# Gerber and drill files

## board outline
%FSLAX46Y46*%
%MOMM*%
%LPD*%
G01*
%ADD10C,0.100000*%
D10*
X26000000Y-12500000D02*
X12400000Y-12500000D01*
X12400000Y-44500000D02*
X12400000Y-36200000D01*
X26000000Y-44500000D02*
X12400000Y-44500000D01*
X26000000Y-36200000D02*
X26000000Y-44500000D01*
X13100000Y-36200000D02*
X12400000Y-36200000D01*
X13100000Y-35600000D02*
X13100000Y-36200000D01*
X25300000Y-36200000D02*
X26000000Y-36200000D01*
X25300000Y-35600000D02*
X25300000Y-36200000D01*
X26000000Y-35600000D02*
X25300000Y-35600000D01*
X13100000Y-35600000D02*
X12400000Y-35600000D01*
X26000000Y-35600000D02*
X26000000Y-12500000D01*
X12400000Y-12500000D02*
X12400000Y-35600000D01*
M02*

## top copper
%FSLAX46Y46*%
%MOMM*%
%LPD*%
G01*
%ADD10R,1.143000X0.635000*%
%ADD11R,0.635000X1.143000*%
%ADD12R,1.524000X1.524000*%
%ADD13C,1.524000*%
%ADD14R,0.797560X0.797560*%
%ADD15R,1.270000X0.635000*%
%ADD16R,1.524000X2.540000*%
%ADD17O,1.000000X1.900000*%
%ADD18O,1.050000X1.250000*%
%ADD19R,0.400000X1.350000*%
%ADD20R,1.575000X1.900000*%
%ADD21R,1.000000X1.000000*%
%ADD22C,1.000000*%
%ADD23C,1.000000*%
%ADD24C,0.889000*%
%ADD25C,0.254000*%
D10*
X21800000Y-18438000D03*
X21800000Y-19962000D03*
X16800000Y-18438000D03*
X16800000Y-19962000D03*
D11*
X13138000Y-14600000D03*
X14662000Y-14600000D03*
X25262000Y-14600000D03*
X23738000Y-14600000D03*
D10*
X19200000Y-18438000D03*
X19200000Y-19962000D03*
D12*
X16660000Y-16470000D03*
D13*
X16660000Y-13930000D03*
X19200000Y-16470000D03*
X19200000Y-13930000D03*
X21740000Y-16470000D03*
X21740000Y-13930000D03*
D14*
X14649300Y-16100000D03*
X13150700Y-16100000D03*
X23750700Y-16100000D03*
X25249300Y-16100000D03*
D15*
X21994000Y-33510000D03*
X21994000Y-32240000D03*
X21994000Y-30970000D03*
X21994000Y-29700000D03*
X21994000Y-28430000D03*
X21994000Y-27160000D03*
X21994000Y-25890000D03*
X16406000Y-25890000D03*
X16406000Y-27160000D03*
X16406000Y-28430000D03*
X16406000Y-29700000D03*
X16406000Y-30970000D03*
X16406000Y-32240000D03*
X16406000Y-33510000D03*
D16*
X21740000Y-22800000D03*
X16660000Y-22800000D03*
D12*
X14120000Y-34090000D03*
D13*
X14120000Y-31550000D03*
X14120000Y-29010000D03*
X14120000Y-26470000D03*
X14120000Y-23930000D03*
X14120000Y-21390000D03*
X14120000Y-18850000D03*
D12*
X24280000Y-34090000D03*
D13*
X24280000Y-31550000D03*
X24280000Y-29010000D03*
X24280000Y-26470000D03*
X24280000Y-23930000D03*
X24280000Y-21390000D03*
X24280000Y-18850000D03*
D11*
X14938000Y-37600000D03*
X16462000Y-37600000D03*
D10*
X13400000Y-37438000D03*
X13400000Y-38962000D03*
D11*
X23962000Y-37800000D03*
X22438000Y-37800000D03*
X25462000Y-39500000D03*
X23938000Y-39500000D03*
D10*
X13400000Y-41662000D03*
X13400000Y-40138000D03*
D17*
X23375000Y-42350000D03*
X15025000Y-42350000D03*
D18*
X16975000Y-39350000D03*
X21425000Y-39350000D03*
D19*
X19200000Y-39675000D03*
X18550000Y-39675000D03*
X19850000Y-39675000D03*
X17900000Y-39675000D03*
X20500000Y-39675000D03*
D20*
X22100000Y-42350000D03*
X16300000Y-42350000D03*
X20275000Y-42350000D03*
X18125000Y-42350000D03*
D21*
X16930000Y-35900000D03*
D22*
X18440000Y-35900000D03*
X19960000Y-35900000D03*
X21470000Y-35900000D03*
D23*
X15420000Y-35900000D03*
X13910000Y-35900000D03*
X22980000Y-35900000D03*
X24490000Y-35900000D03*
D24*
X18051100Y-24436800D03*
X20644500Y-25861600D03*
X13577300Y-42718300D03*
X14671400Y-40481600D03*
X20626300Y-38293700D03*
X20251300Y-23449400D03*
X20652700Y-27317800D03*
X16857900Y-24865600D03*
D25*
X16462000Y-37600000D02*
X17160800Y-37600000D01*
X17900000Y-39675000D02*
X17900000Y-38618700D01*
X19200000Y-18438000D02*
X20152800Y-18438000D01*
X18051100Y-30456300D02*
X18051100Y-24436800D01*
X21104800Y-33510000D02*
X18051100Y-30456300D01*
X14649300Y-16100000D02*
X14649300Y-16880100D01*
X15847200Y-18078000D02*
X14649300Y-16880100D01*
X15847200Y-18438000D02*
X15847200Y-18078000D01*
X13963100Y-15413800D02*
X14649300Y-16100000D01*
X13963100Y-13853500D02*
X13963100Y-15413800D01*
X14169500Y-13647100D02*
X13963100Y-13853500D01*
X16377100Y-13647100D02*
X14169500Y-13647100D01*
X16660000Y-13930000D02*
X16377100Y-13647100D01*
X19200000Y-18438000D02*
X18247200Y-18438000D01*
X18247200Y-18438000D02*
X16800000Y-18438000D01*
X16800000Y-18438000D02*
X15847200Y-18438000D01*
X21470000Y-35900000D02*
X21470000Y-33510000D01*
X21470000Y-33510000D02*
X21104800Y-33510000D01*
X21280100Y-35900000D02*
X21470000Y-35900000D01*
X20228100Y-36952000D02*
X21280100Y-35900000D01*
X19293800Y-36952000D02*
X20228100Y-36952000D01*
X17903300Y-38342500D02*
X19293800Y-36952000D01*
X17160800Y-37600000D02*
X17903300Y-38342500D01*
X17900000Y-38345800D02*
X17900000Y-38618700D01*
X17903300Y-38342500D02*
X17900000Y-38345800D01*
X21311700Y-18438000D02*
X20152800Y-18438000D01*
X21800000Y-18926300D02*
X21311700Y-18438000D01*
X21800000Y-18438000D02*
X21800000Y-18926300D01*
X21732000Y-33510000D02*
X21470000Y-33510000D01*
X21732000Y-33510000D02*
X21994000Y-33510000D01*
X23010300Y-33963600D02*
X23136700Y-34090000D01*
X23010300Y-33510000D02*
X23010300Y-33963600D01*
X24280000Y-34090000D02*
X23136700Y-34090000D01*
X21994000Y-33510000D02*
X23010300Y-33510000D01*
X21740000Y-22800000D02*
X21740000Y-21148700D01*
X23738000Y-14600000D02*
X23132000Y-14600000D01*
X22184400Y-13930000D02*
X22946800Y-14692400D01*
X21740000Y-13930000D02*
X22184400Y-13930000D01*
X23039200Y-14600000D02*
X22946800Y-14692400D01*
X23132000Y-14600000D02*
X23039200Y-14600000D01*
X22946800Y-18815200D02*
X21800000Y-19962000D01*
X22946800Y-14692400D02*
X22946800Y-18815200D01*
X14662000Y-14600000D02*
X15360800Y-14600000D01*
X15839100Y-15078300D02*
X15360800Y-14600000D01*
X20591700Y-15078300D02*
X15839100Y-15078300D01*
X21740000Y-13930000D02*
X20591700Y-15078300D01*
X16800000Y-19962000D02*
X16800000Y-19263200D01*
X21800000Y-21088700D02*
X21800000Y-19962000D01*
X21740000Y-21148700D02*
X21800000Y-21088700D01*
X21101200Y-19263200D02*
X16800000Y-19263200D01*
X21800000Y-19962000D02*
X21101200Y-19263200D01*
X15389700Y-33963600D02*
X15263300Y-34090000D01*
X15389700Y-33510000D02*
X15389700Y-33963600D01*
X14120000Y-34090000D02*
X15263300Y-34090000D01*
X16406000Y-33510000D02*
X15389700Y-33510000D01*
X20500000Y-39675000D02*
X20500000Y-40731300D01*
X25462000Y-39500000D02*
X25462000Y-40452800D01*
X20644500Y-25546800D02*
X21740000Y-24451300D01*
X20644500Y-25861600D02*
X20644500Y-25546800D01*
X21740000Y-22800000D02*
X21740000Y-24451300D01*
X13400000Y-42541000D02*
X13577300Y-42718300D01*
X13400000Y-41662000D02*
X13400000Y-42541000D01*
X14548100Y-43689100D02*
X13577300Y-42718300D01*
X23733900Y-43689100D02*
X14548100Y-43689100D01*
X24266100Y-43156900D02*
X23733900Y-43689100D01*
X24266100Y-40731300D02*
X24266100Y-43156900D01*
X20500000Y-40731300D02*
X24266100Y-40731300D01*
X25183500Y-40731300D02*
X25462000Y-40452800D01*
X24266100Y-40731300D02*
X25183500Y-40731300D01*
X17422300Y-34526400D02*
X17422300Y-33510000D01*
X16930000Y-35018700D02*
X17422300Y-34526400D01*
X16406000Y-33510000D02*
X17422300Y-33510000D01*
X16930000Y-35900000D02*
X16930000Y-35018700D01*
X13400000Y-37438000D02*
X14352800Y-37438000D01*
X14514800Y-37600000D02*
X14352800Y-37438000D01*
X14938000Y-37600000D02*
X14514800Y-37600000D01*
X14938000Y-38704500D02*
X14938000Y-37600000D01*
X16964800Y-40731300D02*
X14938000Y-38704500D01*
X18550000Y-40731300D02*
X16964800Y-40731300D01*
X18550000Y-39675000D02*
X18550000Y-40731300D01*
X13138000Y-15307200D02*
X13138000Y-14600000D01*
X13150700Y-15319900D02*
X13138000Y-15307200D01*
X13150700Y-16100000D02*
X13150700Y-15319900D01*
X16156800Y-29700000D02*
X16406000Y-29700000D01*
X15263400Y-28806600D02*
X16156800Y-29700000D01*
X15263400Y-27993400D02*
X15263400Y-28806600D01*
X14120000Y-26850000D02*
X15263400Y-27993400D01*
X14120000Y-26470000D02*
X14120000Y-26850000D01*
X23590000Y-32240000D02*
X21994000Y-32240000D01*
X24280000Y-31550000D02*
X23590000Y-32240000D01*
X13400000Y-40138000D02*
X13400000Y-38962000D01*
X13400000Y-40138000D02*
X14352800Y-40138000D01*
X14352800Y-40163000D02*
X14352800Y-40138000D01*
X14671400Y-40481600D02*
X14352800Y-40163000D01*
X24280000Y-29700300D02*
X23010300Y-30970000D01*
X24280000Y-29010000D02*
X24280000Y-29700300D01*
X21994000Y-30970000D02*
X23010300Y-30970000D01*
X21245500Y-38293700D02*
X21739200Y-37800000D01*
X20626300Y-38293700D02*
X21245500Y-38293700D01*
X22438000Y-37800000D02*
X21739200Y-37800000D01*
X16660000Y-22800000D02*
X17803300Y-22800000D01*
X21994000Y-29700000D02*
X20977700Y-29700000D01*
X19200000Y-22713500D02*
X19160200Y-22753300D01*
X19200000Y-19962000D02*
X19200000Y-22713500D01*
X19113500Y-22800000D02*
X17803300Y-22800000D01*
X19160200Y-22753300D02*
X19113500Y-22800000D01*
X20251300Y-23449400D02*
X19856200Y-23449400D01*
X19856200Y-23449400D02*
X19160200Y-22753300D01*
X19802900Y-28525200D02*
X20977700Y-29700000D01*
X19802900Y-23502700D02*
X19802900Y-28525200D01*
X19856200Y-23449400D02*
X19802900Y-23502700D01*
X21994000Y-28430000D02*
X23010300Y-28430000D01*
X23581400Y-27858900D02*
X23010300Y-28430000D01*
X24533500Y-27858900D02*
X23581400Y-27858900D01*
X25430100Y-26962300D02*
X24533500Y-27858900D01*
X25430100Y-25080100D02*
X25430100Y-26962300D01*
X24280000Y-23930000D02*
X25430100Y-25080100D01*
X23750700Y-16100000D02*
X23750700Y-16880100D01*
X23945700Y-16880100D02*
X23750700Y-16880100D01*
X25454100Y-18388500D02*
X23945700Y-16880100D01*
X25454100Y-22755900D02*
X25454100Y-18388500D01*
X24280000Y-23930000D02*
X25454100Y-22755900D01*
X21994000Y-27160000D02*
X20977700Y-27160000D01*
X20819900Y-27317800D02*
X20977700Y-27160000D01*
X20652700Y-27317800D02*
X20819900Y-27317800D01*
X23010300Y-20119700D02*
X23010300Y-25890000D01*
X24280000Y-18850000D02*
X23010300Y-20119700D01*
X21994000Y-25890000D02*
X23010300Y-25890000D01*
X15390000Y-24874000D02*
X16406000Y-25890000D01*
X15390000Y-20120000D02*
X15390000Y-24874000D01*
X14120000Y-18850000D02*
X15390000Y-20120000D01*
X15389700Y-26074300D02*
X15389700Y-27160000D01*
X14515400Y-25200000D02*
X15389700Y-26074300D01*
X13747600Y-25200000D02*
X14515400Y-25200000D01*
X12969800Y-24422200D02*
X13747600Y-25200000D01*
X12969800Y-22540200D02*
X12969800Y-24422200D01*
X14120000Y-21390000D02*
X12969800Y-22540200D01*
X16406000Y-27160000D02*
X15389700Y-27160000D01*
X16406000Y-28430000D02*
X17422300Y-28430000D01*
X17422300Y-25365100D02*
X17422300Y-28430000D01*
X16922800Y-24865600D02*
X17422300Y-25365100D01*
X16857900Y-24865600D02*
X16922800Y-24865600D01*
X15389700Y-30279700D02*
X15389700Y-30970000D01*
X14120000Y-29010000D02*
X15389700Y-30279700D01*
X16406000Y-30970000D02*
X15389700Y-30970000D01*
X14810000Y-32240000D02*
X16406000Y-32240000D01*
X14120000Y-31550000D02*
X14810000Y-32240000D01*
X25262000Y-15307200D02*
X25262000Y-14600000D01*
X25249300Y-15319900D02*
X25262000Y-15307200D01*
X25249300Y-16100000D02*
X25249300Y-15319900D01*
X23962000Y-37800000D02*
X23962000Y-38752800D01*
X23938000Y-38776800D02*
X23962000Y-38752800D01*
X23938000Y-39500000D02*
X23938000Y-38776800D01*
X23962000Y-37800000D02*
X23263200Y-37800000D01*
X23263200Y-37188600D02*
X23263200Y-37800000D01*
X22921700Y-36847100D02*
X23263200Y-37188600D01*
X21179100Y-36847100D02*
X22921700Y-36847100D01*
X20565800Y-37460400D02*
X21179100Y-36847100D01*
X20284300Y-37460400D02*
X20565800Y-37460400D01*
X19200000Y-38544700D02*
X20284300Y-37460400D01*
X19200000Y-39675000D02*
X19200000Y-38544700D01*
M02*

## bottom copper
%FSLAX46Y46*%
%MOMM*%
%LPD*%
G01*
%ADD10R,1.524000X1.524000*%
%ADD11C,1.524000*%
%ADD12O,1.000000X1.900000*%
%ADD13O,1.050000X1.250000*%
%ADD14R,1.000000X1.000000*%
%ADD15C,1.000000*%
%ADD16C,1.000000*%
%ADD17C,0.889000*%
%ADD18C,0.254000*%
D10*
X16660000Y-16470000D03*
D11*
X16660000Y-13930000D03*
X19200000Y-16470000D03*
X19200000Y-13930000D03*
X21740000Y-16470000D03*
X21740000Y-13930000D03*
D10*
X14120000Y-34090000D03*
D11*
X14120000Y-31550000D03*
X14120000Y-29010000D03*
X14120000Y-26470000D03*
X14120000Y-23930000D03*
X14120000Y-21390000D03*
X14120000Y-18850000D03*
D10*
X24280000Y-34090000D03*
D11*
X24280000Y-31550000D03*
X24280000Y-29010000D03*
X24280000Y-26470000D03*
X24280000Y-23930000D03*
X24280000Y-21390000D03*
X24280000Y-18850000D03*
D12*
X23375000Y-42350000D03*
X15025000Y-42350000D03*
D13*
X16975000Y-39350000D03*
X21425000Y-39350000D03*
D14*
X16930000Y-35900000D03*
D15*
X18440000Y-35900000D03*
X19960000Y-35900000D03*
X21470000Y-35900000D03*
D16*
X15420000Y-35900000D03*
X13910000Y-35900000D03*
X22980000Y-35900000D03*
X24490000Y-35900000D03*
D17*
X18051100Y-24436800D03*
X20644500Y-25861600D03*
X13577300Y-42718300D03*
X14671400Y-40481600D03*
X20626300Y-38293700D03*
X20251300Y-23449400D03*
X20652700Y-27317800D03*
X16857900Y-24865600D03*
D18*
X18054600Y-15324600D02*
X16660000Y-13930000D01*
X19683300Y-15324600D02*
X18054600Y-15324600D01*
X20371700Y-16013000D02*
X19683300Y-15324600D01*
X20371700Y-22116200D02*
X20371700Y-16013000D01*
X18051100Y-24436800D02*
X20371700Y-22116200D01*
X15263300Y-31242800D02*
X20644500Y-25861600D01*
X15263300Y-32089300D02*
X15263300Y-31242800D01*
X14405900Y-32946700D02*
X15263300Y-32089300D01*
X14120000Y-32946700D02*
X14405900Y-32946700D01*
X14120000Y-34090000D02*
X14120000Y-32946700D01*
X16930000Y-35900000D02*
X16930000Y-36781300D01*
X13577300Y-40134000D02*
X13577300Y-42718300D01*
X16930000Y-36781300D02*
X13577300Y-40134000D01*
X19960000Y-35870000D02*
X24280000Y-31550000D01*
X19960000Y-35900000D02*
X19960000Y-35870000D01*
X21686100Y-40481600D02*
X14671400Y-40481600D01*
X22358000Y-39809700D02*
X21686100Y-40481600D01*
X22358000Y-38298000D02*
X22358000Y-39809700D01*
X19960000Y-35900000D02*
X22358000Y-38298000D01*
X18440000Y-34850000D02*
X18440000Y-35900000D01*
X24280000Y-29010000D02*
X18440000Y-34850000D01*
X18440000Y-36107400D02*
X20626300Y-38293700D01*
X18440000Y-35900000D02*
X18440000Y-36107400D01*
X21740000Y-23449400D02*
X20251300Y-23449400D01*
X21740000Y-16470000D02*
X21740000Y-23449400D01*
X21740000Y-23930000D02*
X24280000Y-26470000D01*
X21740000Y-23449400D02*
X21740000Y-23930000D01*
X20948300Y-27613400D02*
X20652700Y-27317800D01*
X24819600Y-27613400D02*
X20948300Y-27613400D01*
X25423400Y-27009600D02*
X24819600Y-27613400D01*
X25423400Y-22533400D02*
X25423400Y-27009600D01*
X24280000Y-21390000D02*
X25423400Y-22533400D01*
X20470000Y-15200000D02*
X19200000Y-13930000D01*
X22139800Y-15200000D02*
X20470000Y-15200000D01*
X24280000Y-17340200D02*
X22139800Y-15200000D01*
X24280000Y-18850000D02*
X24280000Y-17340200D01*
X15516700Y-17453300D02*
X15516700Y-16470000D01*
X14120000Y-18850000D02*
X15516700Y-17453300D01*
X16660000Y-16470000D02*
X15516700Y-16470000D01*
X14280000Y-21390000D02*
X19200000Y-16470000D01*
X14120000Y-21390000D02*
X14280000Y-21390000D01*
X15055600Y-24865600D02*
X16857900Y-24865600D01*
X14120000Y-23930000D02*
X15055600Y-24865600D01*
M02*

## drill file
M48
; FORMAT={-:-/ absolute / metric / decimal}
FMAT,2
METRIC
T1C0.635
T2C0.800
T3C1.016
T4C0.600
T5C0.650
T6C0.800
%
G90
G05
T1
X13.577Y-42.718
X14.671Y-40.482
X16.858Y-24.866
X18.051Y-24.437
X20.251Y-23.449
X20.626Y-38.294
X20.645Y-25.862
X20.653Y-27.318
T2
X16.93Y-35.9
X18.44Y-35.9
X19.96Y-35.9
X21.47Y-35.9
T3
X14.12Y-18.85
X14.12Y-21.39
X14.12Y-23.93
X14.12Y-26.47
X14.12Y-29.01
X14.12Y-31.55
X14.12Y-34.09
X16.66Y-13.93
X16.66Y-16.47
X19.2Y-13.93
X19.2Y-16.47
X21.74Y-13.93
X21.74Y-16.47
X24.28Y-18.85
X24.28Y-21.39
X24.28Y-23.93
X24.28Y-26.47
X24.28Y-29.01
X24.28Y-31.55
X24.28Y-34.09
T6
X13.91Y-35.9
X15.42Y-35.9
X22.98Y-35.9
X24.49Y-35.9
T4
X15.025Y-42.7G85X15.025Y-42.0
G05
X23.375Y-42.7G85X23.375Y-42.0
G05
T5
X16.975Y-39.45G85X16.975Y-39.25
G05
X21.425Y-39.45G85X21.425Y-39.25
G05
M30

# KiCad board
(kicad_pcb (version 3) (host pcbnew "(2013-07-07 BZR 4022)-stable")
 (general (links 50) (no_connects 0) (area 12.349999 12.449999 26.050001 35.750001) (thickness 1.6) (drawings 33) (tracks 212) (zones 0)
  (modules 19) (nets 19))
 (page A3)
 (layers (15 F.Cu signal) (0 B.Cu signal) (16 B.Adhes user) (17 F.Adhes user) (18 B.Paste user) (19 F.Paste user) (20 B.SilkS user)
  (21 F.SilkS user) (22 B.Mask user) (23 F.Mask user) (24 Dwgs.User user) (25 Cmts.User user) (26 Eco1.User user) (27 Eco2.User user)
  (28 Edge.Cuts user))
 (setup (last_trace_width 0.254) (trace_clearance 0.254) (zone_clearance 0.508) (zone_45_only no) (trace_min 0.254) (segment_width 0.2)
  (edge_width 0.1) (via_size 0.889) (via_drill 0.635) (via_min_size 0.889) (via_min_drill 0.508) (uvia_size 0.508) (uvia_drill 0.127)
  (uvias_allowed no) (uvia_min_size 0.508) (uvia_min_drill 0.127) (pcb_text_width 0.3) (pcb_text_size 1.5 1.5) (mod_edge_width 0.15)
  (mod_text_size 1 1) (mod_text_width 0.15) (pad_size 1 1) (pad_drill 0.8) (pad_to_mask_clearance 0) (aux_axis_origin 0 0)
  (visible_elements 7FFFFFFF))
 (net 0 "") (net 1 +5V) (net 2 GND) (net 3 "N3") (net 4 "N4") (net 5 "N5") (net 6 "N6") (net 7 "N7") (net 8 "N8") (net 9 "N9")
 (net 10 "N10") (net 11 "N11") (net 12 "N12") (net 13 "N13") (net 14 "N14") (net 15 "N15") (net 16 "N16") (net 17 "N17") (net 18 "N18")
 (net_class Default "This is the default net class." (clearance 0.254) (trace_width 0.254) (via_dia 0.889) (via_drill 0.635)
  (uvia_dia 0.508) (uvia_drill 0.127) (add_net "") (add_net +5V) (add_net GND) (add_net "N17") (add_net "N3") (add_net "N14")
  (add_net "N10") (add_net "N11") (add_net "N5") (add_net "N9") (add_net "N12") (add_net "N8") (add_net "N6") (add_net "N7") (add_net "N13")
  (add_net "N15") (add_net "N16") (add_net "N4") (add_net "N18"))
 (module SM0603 (layer F.Cu) (at 21.8 19.2 270)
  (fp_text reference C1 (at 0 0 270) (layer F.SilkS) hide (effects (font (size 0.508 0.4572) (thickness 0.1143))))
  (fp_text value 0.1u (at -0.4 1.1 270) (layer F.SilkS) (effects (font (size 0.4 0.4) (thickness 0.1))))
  (pad 1 smd rect (at -0.762 0 270) (size 0.635 1.143) (layers F.Cu F.Paste F.Mask) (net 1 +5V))
  (pad 2 smd rect (at 0.762 0 270) (size 0.635 1.143) (layers F.Cu F.Paste F.Mask) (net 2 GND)))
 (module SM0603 (layer F.Cu) (at 16.8 19.2 270)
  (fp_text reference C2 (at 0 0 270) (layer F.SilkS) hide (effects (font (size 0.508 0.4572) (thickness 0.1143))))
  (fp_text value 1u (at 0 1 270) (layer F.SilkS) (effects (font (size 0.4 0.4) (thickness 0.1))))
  (pad 1 smd rect (at -0.762 0 270) (size 0.635 1.143) (layers F.Cu F.Paste F.Mask) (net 1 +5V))
  (pad 2 smd rect (at 0.762 0 270) (size 0.635 1.143) (layers F.Cu F.Paste F.Mask) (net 2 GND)))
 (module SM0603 (layer F.Cu) (at 13.9 14.6)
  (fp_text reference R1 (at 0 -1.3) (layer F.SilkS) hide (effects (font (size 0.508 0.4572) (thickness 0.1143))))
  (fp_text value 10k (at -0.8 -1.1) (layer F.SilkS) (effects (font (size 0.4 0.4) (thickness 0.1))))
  (pad 1 smd rect (at -0.762 0) (size 0.635 1.143) (layers F.Cu F.Paste F.Mask) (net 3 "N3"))
  (pad 2 smd rect (at 0.762 0) (size 0.635 1.143) (layers F.Cu F.Paste F.Mask) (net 2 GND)))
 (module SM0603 (layer F.Cu) (at 24.5 14.6 180)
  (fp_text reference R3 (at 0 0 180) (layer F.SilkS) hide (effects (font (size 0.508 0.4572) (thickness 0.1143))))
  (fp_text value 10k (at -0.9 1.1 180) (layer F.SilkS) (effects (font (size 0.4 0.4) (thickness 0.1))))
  (pad 1 smd rect (at -0.762 0 180) (size 0.635 1.143) (layers F.Cu F.Paste F.Mask) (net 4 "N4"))
  (pad 2 smd rect (at 0.762 0 180) (size 0.635 1.143) (layers F.Cu F.Paste F.Mask) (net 2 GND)))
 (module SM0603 (layer F.Cu) (at 19.2 19.2 270)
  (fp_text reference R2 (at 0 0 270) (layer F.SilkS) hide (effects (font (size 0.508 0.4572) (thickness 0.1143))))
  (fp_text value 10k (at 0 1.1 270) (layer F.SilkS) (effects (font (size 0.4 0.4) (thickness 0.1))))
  (pad 1 smd rect (at -0.762 0 270) (size 0.635 1.143) (layers F.Cu F.Paste F.Mask) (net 1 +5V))
  (pad 2 smd rect (at 0.762 0 270) (size 0.635 1.143) (layers F.Cu F.Paste F.Mask) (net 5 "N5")))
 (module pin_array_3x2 (layer F.Cu) (at 19.2 15.2)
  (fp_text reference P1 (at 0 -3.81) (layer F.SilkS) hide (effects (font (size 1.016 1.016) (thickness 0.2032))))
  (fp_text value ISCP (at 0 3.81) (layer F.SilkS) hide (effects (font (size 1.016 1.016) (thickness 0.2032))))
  (pad 1 thru_hole rect (at -2.54 1.27) (size 1.524 1.524) (drill 1.016) (layers *.Cu *.Mask F.SilkS) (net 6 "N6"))
  (pad 2 thru_hole circle (at -2.54 -1.27) (size 1.524 1.524) (drill 1.016) (layers *.Cu *.Mask F.SilkS) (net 1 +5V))
  (pad 3 thru_hole circle (at 0 1.27) (size 1.524 1.524) (drill 1.016) (layers *.Cu *.Mask F.SilkS) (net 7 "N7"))
  (pad 4 thru_hole circle (at 0 -1.27) (size 1.524 1.524) (drill 1.016) (layers *.Cu *.Mask F.SilkS) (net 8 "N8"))
  (pad 5 thru_hole circle (at 2.54 1.27) (size 1.524 1.524) (drill 1.016) (layers *.Cu *.Mask F.SilkS) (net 5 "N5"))
  (pad 6 thru_hole circle (at 2.54 -1.27) (size 1.524 1.524) (drill 1.016) (layers *.Cu *.Mask F.SilkS) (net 2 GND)))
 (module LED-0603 (layer F.Cu) (at 13.9 16.1 180)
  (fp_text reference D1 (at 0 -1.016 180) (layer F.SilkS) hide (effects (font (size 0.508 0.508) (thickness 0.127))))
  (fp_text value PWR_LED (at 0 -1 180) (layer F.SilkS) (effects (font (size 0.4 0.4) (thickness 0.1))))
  (pad 1 smd rect (at -0.7493 0 180) (size 0.79756 0.79756) (layers F.Cu F.Paste F.Mask) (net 1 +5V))
  (pad 2 smd rect (at 0.7493 0 180) (size 0.79756 0.79756) (layers F.Cu F.Paste F.Mask) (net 3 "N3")))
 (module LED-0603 (layer F.Cu) (at 24.5 16.1)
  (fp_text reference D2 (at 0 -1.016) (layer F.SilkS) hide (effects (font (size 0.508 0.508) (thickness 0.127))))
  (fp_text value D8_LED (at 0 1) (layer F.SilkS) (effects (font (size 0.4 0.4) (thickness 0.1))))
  (pad 1 smd rect (at -0.7493 0) (size 0.79756 0.79756) (layers F.Cu F.Paste F.Mask) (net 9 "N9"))
  (pad 2 smd rect (at 0.7493 0) (size 0.79756 0.79756) (layers F.Cu F.Paste F.Mask) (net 4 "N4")))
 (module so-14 (layer F.Cu) (at 19.2 29.7 90)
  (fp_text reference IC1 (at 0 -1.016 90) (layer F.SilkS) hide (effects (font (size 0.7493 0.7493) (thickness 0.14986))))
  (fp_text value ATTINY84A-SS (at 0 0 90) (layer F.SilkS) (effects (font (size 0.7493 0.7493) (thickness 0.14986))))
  (pad 1 smd rect (at -3.81 2.794 90) (size 0.635 1.27) (layers F.Cu F.Paste F.Mask) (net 1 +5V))
  (pad 2 smd rect (at -2.54 2.794 90) (size 0.635 1.27) (layers F.Cu F.Paste F.Mask) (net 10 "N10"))
  (pad 3 smd rect (at -1.27 2.794 90) (size 0.635 1.27) (layers F.Cu F.Paste F.Mask) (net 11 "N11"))
  (pad 4 smd rect (at 0 2.794 90) (size 0.635 1.27) (layers F.Cu F.Paste F.Mask) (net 5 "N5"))
  (pad 5 smd rect (at 1.27 2.794 90) (size 0.635 1.27) (layers F.Cu F.Paste F.Mask) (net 9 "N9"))
  (pad 6 smd rect (at 2.54 2.794 90) (size 0.635 1.27) (layers F.Cu F.Paste F.Mask) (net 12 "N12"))
  (pad 7 smd rect (at 3.81 2.794 90) (size 0.635 1.27) (layers F.Cu F.Paste F.Mask) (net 8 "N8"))
  (pad 8 smd rect (at 3.81 -2.794 90) (size 0.635 1.27) (layers F.Cu F.Paste F.Mask) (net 6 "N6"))
  (pad 9 smd rect (at 2.54 -2.794 90) (size 0.635 1.27) (layers F.Cu F.Paste F.Mask) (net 7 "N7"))
  (pad 10 smd rect (at 1.27 -2.794 90) (size 0.635 1.27) (layers F.Cu F.Paste F.Mask) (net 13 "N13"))
  (pad 11 smd rect (at 0 -2.794 90) (size 0.635 1.27) (layers F.Cu F.Paste F.Mask) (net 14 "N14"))
  (pad 12 smd rect (at -1.27 -2.794 90) (size 0.635 1.27) (layers F.Cu F.Paste F.Mask) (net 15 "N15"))
  (pad 13 smd rect (at -2.54 -2.794 90) (size 0.635 1.27) (layers F.Cu F.Paste F.Mask) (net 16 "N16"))
  (pad 14 smd rect (at -3.81 -2.794 90) (size 0.635 1.27) (layers F.Cu F.Paste F.Mask) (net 2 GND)))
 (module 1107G (layer F.Cu) (at 19.2 22.8)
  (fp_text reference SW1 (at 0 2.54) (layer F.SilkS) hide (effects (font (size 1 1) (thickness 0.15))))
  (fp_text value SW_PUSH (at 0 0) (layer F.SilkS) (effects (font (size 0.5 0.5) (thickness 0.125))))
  (pad 1 smd rect (at 2.54 0) (size 1.524 2.54) (layers F.Cu F.Paste F.Mask) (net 2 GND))
  (pad 2 smd rect (at -2.54 0) (size 1.524 2.54) (layers F.Cu F.Paste F.Mask) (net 5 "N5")))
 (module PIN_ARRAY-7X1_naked (layer F.Cu) (at 14.12 26.47 90)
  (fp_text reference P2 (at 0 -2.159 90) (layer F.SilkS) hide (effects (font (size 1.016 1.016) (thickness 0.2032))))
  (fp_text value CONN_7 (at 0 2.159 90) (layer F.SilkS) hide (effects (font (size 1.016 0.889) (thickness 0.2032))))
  (pad 1 thru_hole rect (at -7.62 0 90) (size 1.524 1.524) (drill 1.016) (layers *.Cu *.Mask F.SilkS) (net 2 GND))
  (pad 2 thru_hole circle (at -5.08 0 90) (size 1.524 1.524) (drill 1.016) (layers *.Cu *.Mask F.SilkS) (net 16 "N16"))
  (pad 3 thru_hole circle (at -2.54 0 90) (size 1.524 1.524) (drill 1.016) (layers *.Cu *.Mask F.SilkS) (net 15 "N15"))
  (pad 4 thru_hole circle (at 0 0 90) (size 1.524 1.524) (drill 1.016) (layers *.Cu *.Mask F.SilkS) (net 14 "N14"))
  (pad 5 thru_hole circle (at 2.54 0 90) (size 1.524 1.524) (drill 1.016) (layers *.Cu *.Mask F.SilkS) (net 13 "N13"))
  (pad 6 thru_hole circle (at 5.08 0 90) (size 1.524 1.524) (drill 1.016) (layers *.Cu *.Mask F.SilkS) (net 7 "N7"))
  (pad 7 thru_hole circle (at 7.62 0 90) (size 1.524 1.524) (drill 1.016) (layers *.Cu *.Mask F.SilkS) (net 6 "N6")))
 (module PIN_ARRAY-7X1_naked (layer F.Cu) (at 24.28 26.47 90)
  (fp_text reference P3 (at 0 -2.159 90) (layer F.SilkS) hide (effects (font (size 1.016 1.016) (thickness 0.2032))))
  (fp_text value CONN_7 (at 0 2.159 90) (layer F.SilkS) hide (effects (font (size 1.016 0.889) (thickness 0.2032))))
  (pad 1 thru_hole rect (at -7.62 0 90) (size 1.524 1.524) (drill 1.016) (layers *.Cu *.Mask F.SilkS) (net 1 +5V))
  (pad 2 thru_hole circle (at -5.08 0 90) (size 1.524 1.524) (drill 1.016) (layers *.Cu *.Mask F.SilkS) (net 10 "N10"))
  (pad 3 thru_hole circle (at -2.54 0 90) (size 1.524 1.524) (drill 1.016) (layers *.Cu *.Mask F.SilkS) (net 11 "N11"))
  (pad 4 thru_hole circle (at 0 0 90) (size 1.524 1.524) (drill 1.016) (layers *.Cu *.Mask F.SilkS) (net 5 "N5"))
  (pad 5 thru_hole circle (at 2.54 0 90) (size 1.524 1.524) (drill 1.016) (layers *.Cu *.Mask F.SilkS) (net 9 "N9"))
  (pad 6 thru_hole circle (at 5.08 0 90) (size 1.524 1.524) (drill 1.016) (layers *.Cu *.Mask F.SilkS) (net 12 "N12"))
  (pad 7 thru_hole circle (at 7.62 0 90) (size 1.524 1.524) (drill 1.016) (layers *.Cu *.Mask F.SilkS) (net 8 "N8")))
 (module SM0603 (layer F.Cu) (at 15.7 37.6)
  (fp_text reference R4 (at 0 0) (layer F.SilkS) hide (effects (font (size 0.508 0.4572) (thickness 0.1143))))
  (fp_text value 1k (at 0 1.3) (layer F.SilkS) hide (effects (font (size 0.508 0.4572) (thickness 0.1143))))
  (pad 1 smd rect (at -0.762 0) (size 0.635 1.143) (layers F.Cu F.Paste F.Mask) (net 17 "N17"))
  (pad 2 smd rect (at 0.762 0) (size 0.635 1.143) (layers F.Cu F.Paste F.Mask) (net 1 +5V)))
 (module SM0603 (layer F.Cu) (at 13.4 38.2 270)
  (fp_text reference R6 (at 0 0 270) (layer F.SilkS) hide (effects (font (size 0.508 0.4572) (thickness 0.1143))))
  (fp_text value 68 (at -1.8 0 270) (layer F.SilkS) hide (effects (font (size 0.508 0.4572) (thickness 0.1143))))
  (pad 1 smd rect (at -0.762 0 270) (size 0.635 1.143) (layers F.Cu F.Paste F.Mask) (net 17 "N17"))
  (pad 2 smd rect (at 0.762 0 270) (size 0.635 1.143) (layers F.Cu F.Paste F.Mask) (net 10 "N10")))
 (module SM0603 (layer F.Cu) (at 23.2 37.8 180)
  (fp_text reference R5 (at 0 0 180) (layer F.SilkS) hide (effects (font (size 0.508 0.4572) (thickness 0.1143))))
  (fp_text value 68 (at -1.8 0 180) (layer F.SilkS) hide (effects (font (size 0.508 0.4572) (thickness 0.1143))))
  (pad 1 smd rect (at -0.762 0 180) (size 0.635 1.143) (layers F.Cu F.Paste F.Mask) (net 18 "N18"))
  (pad 2 smd rect (at 0.762 0 180) (size 0.635 1.143) (layers F.Cu F.Paste F.Mask) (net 11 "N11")))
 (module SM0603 (layer F.Cu) (at 24.7 39.5 180)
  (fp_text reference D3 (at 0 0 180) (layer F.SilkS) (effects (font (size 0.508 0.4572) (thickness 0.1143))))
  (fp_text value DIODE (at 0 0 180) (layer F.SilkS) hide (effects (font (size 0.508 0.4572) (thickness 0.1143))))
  (pad 1 smd rect (at -0.762 0 180) (size 0.635 1.143) (layers F.Cu F.Paste F.Mask) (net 2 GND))
  (pad 2 smd rect (at 0.762 0 180) (size 0.635 1.143) (layers F.Cu F.Paste F.Mask) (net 18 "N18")))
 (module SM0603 (layer F.Cu) (at 13.4 40.9 90)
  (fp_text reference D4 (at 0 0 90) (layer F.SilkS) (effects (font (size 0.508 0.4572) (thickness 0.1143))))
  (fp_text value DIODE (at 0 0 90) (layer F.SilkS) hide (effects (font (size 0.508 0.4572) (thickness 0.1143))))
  (pad 1 smd rect (at -0.762 0 90) (size 0.635 1.143) (layers F.Cu F.Paste F.Mask) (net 2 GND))
  (pad 2 smd rect (at 0.762 0 90) (size 0.635 1.143) (layers F.Cu F.Paste F.Mask) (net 10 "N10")))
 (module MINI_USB (layer F.Cu) (at 19.2 42 180)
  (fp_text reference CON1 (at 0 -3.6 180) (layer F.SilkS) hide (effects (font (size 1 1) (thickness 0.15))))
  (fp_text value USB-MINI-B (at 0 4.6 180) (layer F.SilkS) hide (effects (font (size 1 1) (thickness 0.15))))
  (pad "" np_thru_hole oval (at -4.175 -0.35 180) (size 1 1.9) (drill oval 0.6 1.3) (layers *.Cu *.Mask F.SilkS))
  (pad "" np_thru_hole oval (at 4.175 -0.35 180) (size 1 1.9) (drill oval 0.6 1.3) (layers *.Cu *.Mask F.SilkS))
  (pad "" np_thru_hole oval (at 2.225 2.65 180) (size 1.05 1.25) (drill oval 0.65 0.85) (layers *.Cu *.Mask F.SilkS))
  (pad "" np_thru_hole oval (at -2.225 2.65 180) (size 1.05 1.25) (drill oval 0.65 0.85) (layers *.Cu *.Mask F.SilkS))
  (pad 3 smd rect (at 0 2.325 180) (size 0.4 1.35) (layers F.Cu F.Paste F.Mask) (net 18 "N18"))
  (pad 2 smd rect (at 0.65 2.325 180) (size 0.4 1.35) (layers F.Cu F.Paste F.Mask) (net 17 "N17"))
  (pad 4 smd rect (at -0.65 2.325 180) (size 0.4 1.35) (layers F.Cu F.Paste F.Mask))
  (pad 1 smd rect (at 1.3 2.325 180) (size 0.4 1.35) (layers F.Cu F.Paste F.Mask) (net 1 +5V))
  (pad 5 smd rect (at -1.3 2.325 180) (size 0.4 1.35) (layers F.Cu F.Paste F.Mask) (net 2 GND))
  (pad "" smd rect (at -2.9 -0.35 180) (size 1.575 1.9) (layers F.Cu F.Paste F.Mask))
  (pad "" smd rect (at 2.9 -0.35 180) (size 1.575 1.9) (layers F.Cu F.Paste F.Mask))
  (pad "" smd rect (at -1.075 -0.35 180) (size 1.575 1.9) (layers F.Cu F.Paste F.Mask))
  (pad "" smd rect (at 1.075 -0.35 180) (size 1.575 1.9) (layers F.Cu F.Paste F.Mask)))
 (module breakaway (layer F.Cu) (at 19.2 35.9)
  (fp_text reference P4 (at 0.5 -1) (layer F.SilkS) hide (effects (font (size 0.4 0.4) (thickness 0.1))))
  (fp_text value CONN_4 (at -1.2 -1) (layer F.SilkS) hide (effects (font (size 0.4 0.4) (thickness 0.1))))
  (pad 1 thru_hole rect (at -2.27 0) (size 1 1) (drill 0.8) (layers *.Cu *.Mask F.SilkS) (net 2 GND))
  (pad 2 thru_hole circle (at -0.76 0) (size 1 1) (drill 0.8) (layers *.Cu *.Mask F.SilkS) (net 11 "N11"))
  (pad 3 thru_hole circle (at 0.76 0) (size 1 1) (drill 0.8) (layers *.Cu *.Mask F.SilkS) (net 10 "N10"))
  (pad 4 thru_hole circle (at 2.27 0) (size 1 1) (drill 0.8) (layers *.Cu *.Mask F.SilkS) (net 1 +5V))
  (pad "" np_thru_hole circle (at -3.78 0) (size 1 1) (drill 0.8) (layers *.Cu *.Mask F.SilkS))
  (pad "" np_thru_hole circle (at -5.29 0) (size 1 1) (drill 0.8) (layers *.Cu *.Mask F.SilkS))
  (pad "" np_thru_hole circle (at 3.78 0) (size 1 1) (drill 0.8) (layers *.Cu *.Mask F.SilkS))
  (pad "" np_thru_hole circle (at 5.29 0) (size 1 1) (drill 0.8) (layers *.Cu *.Mask F.SilkS)))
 (gr_line (start 26 12.5) (end 12.4 12.5) (angle 90) (layer Edge.Cuts) (width 0.1))
 (gr_line (start 12.4 44.5) (end 12.4 36.2) (angle 90) (layer Edge.Cuts) (width 0.1))
 (gr_line (start 26 44.5) (end 12.4 44.5) (angle 90) (layer Edge.Cuts) (width 0.1))
 (gr_line (start 26 36.2) (end 26 44.5) (angle 90) (layer Edge.Cuts) (width 0.1))
 (gr_line (start 13.1 36.2) (end 12.4 36.2) (angle 90) (layer Edge.Cuts) (width 0.1))
 (gr_line (start 13.1 35.6) (end 13.1 36.2) (angle 90) (layer Edge.Cuts) (width 0.1))
 (gr_line (start 25.3 36.2) (end 26 36.2) (angle 90) (layer Edge.Cuts) (width 0.1))
 (gr_line (start 25.3 35.6) (end 25.3 36.2) (angle 90) (layer Edge.Cuts) (width 0.1))
 (gr_line (start 26 35.6) (end 25.3 35.6) (angle 90) (layer Edge.Cuts) (width 0.1))
 (gr_line (start 13.1 35.6) (end 12.4 35.6) (angle 90) (layer Edge.Cuts) (width 0.1))
 (gr_line (start 26 35.6) (end 26 12.5) (angle 90) (layer Edge.Cuts) (width 0.1))
 (gr_line (start 12.4 12.5) (end 12.4 35.6) (angle 90) (layer Edge.Cuts) (width 0.1))
 (via (at 18.0511 24.4368) (size 0.889) (layers F.Cu B.Cu) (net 1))
 (segment (start 16.462 37.6) (end 17.1608 37.6) (width 0.254) (layer F.Cu) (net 1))
 (segment (start 17.9 39.675) (end 17.9 38.6187) (width 0.254) (layer F.Cu) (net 1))
 (segment (start 19.2 18.438) (end 20.1528 18.438) (width 0.254) (layer F.Cu) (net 1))
 (segment (start 18.0546 15.3246) (end 16.66 13.93) (width 0.254) (layer B.Cu) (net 1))
 (segment (start 19.6833 15.3246) (end 18.0546 15.3246) (width 0.254) (layer B.Cu) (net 1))
 (segment (start 20.3717 16.013) (end 19.6833 15.3246) (width 0.254) (layer B.Cu) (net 1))
 (segment (start 20.3717 22.1162) (end 20.3717 16.013) (width 0.254) (layer B.Cu) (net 1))
 (segment (start 18.0511 24.4368) (end 20.3717 22.1162) (width 0.254) (layer B.Cu) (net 1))
 (segment (start 18.0511 30.4563) (end 18.0511 24.4368) (width 0.254) (layer F.Cu) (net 1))
 (segment (start 21.1048 33.51) (end 18.0511 30.4563) (width 0.254) (layer F.Cu) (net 1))
 (segment (start 14.6493 16.1) (end 14.6493 16.8801) (width 0.254) (layer F.Cu) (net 1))
 (segment (start 15.8472 18.078) (end 14.6493 16.8801) (width 0.254) (layer F.Cu) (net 1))
 (segment (start 15.8472 18.438) (end 15.8472 18.078) (width 0.254) (layer F.Cu) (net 1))
 (segment (start 13.9631 15.4138) (end 14.6493 16.1) (width 0.254) (layer F.Cu) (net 1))
 (segment (start 13.9631 13.8535) (end 13.9631 15.4138) (width 0.254) (layer F.Cu) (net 1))
 (segment (start 14.1695 13.6471) (end 13.9631 13.8535) (width 0.254) (layer F.Cu) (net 1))
 (segment (start 16.3771 13.6471) (end 14.1695 13.6471) (width 0.254) (layer F.Cu) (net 1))
 (segment (start 16.66 13.93) (end 16.3771 13.6471) (width 0.254) (layer F.Cu) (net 1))
 (segment (start 19.2 18.438) (end 18.2472 18.438) (width 0.254) (layer F.Cu) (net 1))
 (segment (start 18.2472 18.438) (end 16.8 18.438) (width 0.254) (layer F.Cu) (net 1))
 (segment (start 16.8 18.438) (end 15.8472 18.438) (width 0.254) (layer F.Cu) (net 1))
 (segment (start 21.47 35.9) (end 21.47 33.51) (width 0.254) (layer F.Cu) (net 1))
 (segment (start 21.47 33.51) (end 21.1048 33.51) (width 0.254) (layer F.Cu) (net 1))
 (segment (start 21.2801 35.9) (end 21.47 35.9) (width 0.254) (layer F.Cu) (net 1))
 (segment (start 20.2281 36.952) (end 21.2801 35.9) (width 0.254) (layer F.Cu) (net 1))
 (segment (start 19.2938 36.952) (end 20.2281 36.952) (width 0.254) (layer F.Cu) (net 1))
 (segment (start 17.9033 38.3425) (end 19.2938 36.952) (width 0.254) (layer F.Cu) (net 1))
 (segment (start 17.1608 37.6) (end 17.9033 38.3425) (width 0.254) (layer F.Cu) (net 1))
 (segment (start 17.9 38.3458) (end 17.9 38.6187) (width 0.254) (layer F.Cu) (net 1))
 (segment (start 17.9033 38.3425) (end 17.9 38.3458) (width 0.254) (layer F.Cu) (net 1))
 (segment (start 21.3117 18.438) (end 20.1528 18.438) (width 0.254) (layer F.Cu) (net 1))
 (segment (start 21.8 18.9263) (end 21.3117 18.438) (width 0.254) (layer F.Cu) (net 1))
 (segment (start 21.8 18.438) (end 21.8 18.9263) (width 0.254) (layer F.Cu) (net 1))
 (segment (start 21.732 33.51) (end 21.47 33.51) (width 0.254) (layer F.Cu) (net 1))
 (segment (start 21.732 33.51) (end 21.994 33.51) (width 0.254) (layer F.Cu) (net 1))
 (segment (start 23.0103 33.9636) (end 23.1367 34.09) (width 0.254) (layer F.Cu) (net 1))
 (segment (start 23.0103 33.51) (end 23.0103 33.9636) (width 0.254) (layer F.Cu) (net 1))
 (segment (start 24.28 34.09) (end 23.1367 34.09) (width 0.254) (layer F.Cu) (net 1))
 (segment (start 21.994 33.51) (end 23.0103 33.51) (width 0.254) (layer F.Cu) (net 1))
 (via (at 20.6445 25.8616) (size 0.889) (layers F.Cu B.Cu) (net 2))
 (via (at 13.5773 42.7183) (size 0.889) (layers F.Cu B.Cu) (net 2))
 (segment (start 21.74 22.8) (end 21.74 21.1487) (width 0.254) (layer F.Cu) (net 2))
 (segment (start 23.738 14.6) (end 23.132 14.6) (width 0.254) (layer F.Cu) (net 2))
 (segment (start 22.1844 13.93) (end 22.9468 14.6924) (width 0.254) (layer F.Cu) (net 2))
 (segment (start 21.74 13.93) (end 22.1844 13.93) (width 0.254) (layer F.Cu) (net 2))
 (segment (start 23.0392 14.6) (end 22.9468 14.6924) (width 0.254) (layer F.Cu) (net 2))
 (segment (start 23.132 14.6) (end 23.0392 14.6) (width 0.254) (layer F.Cu) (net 2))
 (segment (start 22.9468 18.8152) (end 21.8 19.962) (width 0.254) (layer F.Cu) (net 2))
 (segment (start 22.9468 14.6924) (end 22.9468 18.8152) (width 0.254) (layer F.Cu) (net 2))
 (segment (start 14.662 14.6) (end 15.3608 14.6) (width 0.254) (layer F.Cu) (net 2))
 (segment (start 15.8391 15.0783) (end 15.3608 14.6) (width 0.254) (layer F.Cu) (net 2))
 (segment (start 20.5917 15.0783) (end 15.8391 15.0783) (width 0.254) (layer F.Cu) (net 2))
 (segment (start 21.74 13.93) (end 20.5917 15.0783) (width 0.254) (layer F.Cu) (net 2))
 (segment (start 16.8 19.962) (end 16.8 19.2632) (width 0.254) (layer F.Cu) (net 2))
 (segment (start 21.8 21.0887) (end 21.8 19.962) (width 0.254) (layer F.Cu) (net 2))
 (segment (start 21.74 21.1487) (end 21.8 21.0887) (width 0.254) (layer F.Cu) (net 2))
 (segment (start 21.1012 19.2632) (end 16.8 19.2632) (width 0.254) (layer F.Cu) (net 2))
 (segment (start 21.8 19.962) (end 21.1012 19.2632) (width 0.254) (layer F.Cu) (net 2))
 (segment (start 15.3897 33.9636) (end 15.2633 34.09) (width 0.254) (layer F.Cu) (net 2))
 (segment (start 15.3897 33.51) (end 15.3897 33.9636) (width 0.254) (layer F.Cu) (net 2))
 (segment (start 14.12 34.09) (end 15.2633 34.09) (width 0.254) (layer F.Cu) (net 2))
 (segment (start 16.406 33.51) (end 15.3897 33.51) (width 0.254) (layer F.Cu) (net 2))
 (segment (start 20.5 39.675) (end 20.5 40.7313) (width 0.254) (layer F.Cu) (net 2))
 (segment (start 25.462 39.5) (end 25.462 40.4528) (width 0.254) (layer F.Cu) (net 2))
 (segment (start 15.2633 31.2428) (end 20.6445 25.8616) (width 0.254) (layer B.Cu) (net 2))
 (segment (start 15.2633 32.0893) (end 15.2633 31.2428) (width 0.254) (layer B.Cu) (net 2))
 (segment (start 14.4059 32.9467) (end 15.2633 32.0893) (width 0.254) (layer B.Cu) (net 2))
 (segment (start 14.12 32.9467) (end 14.4059 32.9467) (width 0.254) (layer B.Cu) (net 2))
 (segment (start 20.6445 25.5468) (end 21.74 24.4513) (width 0.254) (layer F.Cu) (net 2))
 (segment (start 20.6445 25.8616) (end 20.6445 25.5468) (width 0.254) (layer F.Cu) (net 2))
 (segment (start 21.74 22.8) (end 21.74 24.4513) (width 0.254) (layer F.Cu) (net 2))
 (segment (start 14.12 34.09) (end 14.12 32.9467) (width 0.254) (layer B.Cu) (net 2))
 (segment (start 16.93 35.9) (end 16.93 36.7813) (width 0.254) (layer B.Cu) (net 2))
 (segment (start 13.5773 40.134) (end 13.5773 42.7183) (width 0.254) (layer B.Cu) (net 2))
 (segment (start 16.93 36.7813) (end 13.5773 40.134) (width 0.254) (layer B.Cu) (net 2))
 (segment (start 13.4 42.541) (end 13.5773 42.7183) (width 0.254) (layer F.Cu) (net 2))
 (segment (start 13.4 41.662) (end 13.4 42.541) (width 0.254) (layer F.Cu) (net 2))
 (segment (start 14.5481 43.6891) (end 13.5773 42.7183) (width 0.254) (layer F.Cu) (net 2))
 (segment (start 23.7339 43.6891) (end 14.5481 43.6891) (width 0.254) (layer F.Cu) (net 2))
 (segment (start 24.2661 43.1569) (end 23.7339 43.6891) (width 0.254) (layer F.Cu) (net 2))
 (segment (start 24.2661 40.7313) (end 24.2661 43.1569) (width 0.254) (layer F.Cu) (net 2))
 (segment (start 20.5 40.7313) (end 24.2661 40.7313) (width 0.254) (layer F.Cu) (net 2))
 (segment (start 25.1835 40.7313) (end 25.462 40.4528) (width 0.254) (layer F.Cu) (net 2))
 (segment (start 24.2661 40.7313) (end 25.1835 40.7313) (width 0.254) (layer F.Cu) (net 2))
 (segment (start 17.4223 34.5264) (end 17.4223 33.51) (width 0.254) (layer F.Cu) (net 2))
 (segment (start 16.93 35.0187) (end 17.4223 34.5264) (width 0.254) (layer F.Cu) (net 2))
 (segment (start 16.406 33.51) (end 17.4223 33.51) (width 0.254) (layer F.Cu) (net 2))
 (segment (start 16.93 35.9) (end 16.93 35.0187) (width 0.254) (layer F.Cu) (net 2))
 (segment (start 13.4 37.438) (end 14.3528 37.438) (width 0.254) (layer F.Cu) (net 17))
 (segment (start 14.5148 37.6) (end 14.3528 37.438) (width 0.254) (layer F.Cu) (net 17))
 (segment (start 14.938 37.6) (end 14.5148 37.6) (width 0.254) (layer F.Cu) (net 17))
 (segment (start 14.938 38.7045) (end 14.938 37.6) (width 0.254) (layer F.Cu) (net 17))
 (segment (start 16.9648 40.7313) (end 14.938 38.7045) (width 0.254) (layer F.Cu) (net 17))
 (segment (start 18.55 40.7313) (end 16.9648 40.7313) (width 0.254) (layer F.Cu) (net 17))
 (segment (start 18.55 39.675) (end 18.55 40.7313) (width 0.254) (layer F.Cu) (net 17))
 (segment (start 13.138 15.3072) (end 13.138 14.6) (width 0.254) (layer F.Cu) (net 3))
 (segment (start 13.1507 15.3199) (end 13.138 15.3072) (width 0.254) (layer F.Cu) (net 3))
 (segment (start 13.1507 16.1) (end 13.1507 15.3199) (width 0.254) (layer F.Cu) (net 3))
 (segment (start 16.1568 29.7) (end 16.406 29.7) (width 0.254) (layer F.Cu) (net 14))
 (segment (start 15.2634 28.8066) (end 16.1568 29.7) (width 0.254) (layer F.Cu) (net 14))
 (segment (start 15.2634 27.9934) (end 15.2634 28.8066) (width 0.254) (layer F.Cu) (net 14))
 (segment (start 14.12 26.85) (end 15.2634 27.9934) (width 0.254) (layer F.Cu) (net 14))
 (segment (start 14.12 26.47) (end 14.12 26.85) (width 0.254) (layer F.Cu) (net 14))
 (via (at 14.6714 40.4816) (size 0.889) (layers F.Cu B.Cu) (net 10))
 (segment (start 23.59 32.24) (end 21.994 32.24) (width 0.254) (layer F.Cu) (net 10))
 (segment (start 24.28 31.55) (end 23.59 32.24) (width 0.254) (layer F.Cu) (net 10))
 (segment (start 13.4 40.138) (end 13.4 38.962) (width 0.254) (layer F.Cu) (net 10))
 (segment (start 13.4 40.138) (end 14.3528 40.138) (width 0.254) (layer F.Cu) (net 10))
 (segment (start 19.96 35.87) (end 24.28 31.55) (width 0.254) (layer B.Cu) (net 10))
 (segment (start 19.96 35.9) (end 19.96 35.87) (width 0.254) (layer B.Cu) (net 10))
 (segment (start 21.6861 40.4816) (end 14.6714 40.4816) (width 0.254) (layer B.Cu) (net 10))
 (segment (start 22.358 39.8097) (end 21.6861 40.4816) (width 0.254) (layer B.Cu) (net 10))
 (segment (start 22.358 38.298) (end 22.358 39.8097) (width 0.254) (layer B.Cu) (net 10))
 (segment (start 19.96 35.9) (end 22.358 38.298) (width 0.254) (layer B.Cu) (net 10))
 (segment (start 14.3528 40.163) (end 14.3528 40.138) (width 0.254) (layer F.Cu) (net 10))
 (segment (start 14.6714 40.4816) (end 14.3528 40.163) (width 0.254) (layer F.Cu) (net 10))
 (via (at 20.6263 38.2937) (size 0.889) (layers F.Cu B.Cu) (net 11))
 (segment (start 24.28 29.7003) (end 23.0103 30.97) (width 0.254) (layer F.Cu) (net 11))
 (segment (start 24.28 29.01) (end 24.28 29.7003) (width 0.254) (layer F.Cu) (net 11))
 (segment (start 21.994 30.97) (end 23.0103 30.97) (width 0.254) (layer F.Cu) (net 11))
 (segment (start 18.44 34.85) (end 18.44 35.9) (width 0.254) (layer B.Cu) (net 11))
 (segment (start 24.28 29.01) (end 18.44 34.85) (width 0.254) (layer B.Cu) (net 11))
 (segment (start 18.44 36.1074) (end 20.6263 38.2937) (width 0.254) (layer B.Cu) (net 11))
 (segment (start 18.44 35.9) (end 18.44 36.1074) (width 0.254) (layer B.Cu) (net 11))
 (segment (start 21.2455 38.2937) (end 21.7392 37.8) (width 0.254) (layer F.Cu) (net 11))
 (segment (start 20.6263 38.2937) (end 21.2455 38.2937) (width 0.254) (layer F.Cu) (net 11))
 (segment (start 22.438 37.8) (end 21.7392 37.8) (width 0.254) (layer F.Cu) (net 11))
 (via (at 20.2513 23.4494) (size 0.889) (layers F.Cu B.Cu) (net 5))
 (segment (start 16.66 22.8) (end 17.8033 22.8) (width 0.254) (layer F.Cu) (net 5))
 (segment (start 21.994 29.7) (end 20.9777 29.7) (width 0.254) (layer F.Cu) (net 5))
 (segment (start 19.2 22.7135) (end 19.1602 22.7533) (width 0.254) (layer F.Cu) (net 5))
 (segment (start 19.2 19.962) (end 19.2 22.7135) (width 0.254) (layer F.Cu) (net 5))
 (segment (start 19.1135 22.8) (end 17.8033 22.8) (width 0.254) (layer F.Cu) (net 5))
 (segment (start 19.1602 22.7533) (end 19.1135 22.8) (width 0.254) (layer F.Cu) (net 5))
 (segment (start 20.2513 23.4494) (end 19.8562 23.4494) (width 0.254) (layer F.Cu) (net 5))
 (segment (start 19.8562 23.4494) (end 19.1602 22.7533) (width 0.254) (layer F.Cu) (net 5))
 (segment (start 21.74 23.4494) (end 20.2513 23.4494) (width 0.254) (layer B.Cu) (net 5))
 (segment (start 21.74 16.47) (end 21.74 23.4494) (width 0.254) (layer B.Cu) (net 5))
 (segment (start 21.74 23.93) (end 24.28 26.47) (width 0.254) (layer B.Cu) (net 5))
 (segment (start 21.74 23.4494) (end 21.74 23.93) (width 0.254) (layer B.Cu) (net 5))
 (segment (start 19.8029 28.5252) (end 20.9777 29.7) (width 0.254) (layer F.Cu) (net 5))
 (segment (start 19.8029 23.5027) (end 19.8029 28.5252) (width 0.254) (layer F.Cu) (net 5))
 (segment (start 19.8562 23.4494) (end 19.8029 23.5027) (width 0.254) (layer F.Cu) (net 5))
 (segment (start 21.994 28.43) (end 23.0103 28.43) (width 0.254) (layer F.Cu) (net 9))
 (segment (start 23.5814 27.8589) (end 23.0103 28.43) (width 0.254) (layer F.Cu) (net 9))
 (segment (start 24.5335 27.8589) (end 23.5814 27.8589) (width 0.254) (layer F.Cu) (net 9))
 (segment (start 25.4301 26.9623) (end 24.5335 27.8589) (width 0.254) (layer F.Cu) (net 9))
 (segment (start 25.4301 25.0801) (end 25.4301 26.9623) (width 0.254) (layer F.Cu) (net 9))
 (segment (start 24.28 23.93) (end 25.4301 25.0801) (width 0.254) (layer F.Cu) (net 9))
 (segment (start 23.7507 16.1) (end 23.7507 16.8801) (width 0.254) (layer F.Cu) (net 9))
 (segment (start 23.9457 16.8801) (end 23.7507 16.8801) (width 0.254) (layer F.Cu) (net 9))
 (segment (start 25.4541 18.3885) (end 23.9457 16.8801) (width 0.254) (layer F.Cu) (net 9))
 (segment (start 25.4541 22.7559) (end 25.4541 18.3885) (width 0.254) (layer F.Cu) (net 9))
 (segment (start 24.28 23.93) (end 25.4541 22.7559) (width 0.254) (layer F.Cu) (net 9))
 (via (at 20.6527 27.3178) (size 0.889) (layers F.Cu B.Cu) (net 12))
 (segment (start 21.994 27.16) (end 20.9777 27.16) (width 0.254) (layer F.Cu) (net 12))
 (segment (start 20.9483 27.6134) (end 20.6527 27.3178) (width 0.254) (layer B.Cu) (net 12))
 (segment (start 24.8196 27.6134) (end 20.9483 27.6134) (width 0.254) (layer B.Cu) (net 12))
 (segment (start 25.4234 27.0096) (end 24.8196 27.6134) (width 0.254) (layer B.Cu) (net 12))
 (segment (start 25.4234 22.5334) (end 25.4234 27.0096) (width 0.254) (layer B.Cu) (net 12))
 (segment (start 24.28 21.39) (end 25.4234 22.5334) (width 0.254) (layer B.Cu) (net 12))
 (segment (start 20.8199 27.3178) (end 20.9777 27.16) (width 0.254) (layer F.Cu) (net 12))
 (segment (start 20.6527 27.3178) (end 20.8199 27.3178) (width 0.254) (layer F.Cu) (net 12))
 (segment (start 23.0103 20.1197) (end 23.0103 25.89) (width 0.254) (layer F.Cu) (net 8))
 (segment (start 24.28 18.85) (end 23.0103 20.1197) (width 0.254) (layer F.Cu) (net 8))
 (segment (start 21.994 25.89) (end 23.0103 25.89) (width 0.254) (layer F.Cu) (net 8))
 (segment (start 20.47 15.2) (end 19.2 13.93) (width 0.254) (layer B.Cu) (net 8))
 (segment (start 22.1398 15.2) (end 20.47 15.2) (width 0.254) (layer B.Cu) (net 8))
 (segment (start 24.28 17.3402) (end 22.1398 15.2) (width 0.254) (layer B.Cu) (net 8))
 (segment (start 24.28 18.85) (end 24.28 17.3402) (width 0.254) (layer B.Cu) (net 8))
 (segment (start 15.5167 17.4533) (end 15.5167 16.47) (width 0.254) (layer B.Cu) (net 6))
 (segment (start 14.12 18.85) (end 15.5167 17.4533) (width 0.254) (layer B.Cu) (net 6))
 (segment (start 16.66 16.47) (end 15.5167 16.47) (width 0.254) (layer B.Cu) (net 6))
 (segment (start 15.39 24.874) (end 16.406 25.89) (width 0.254) (layer F.Cu) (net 6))
 (segment (start 15.39 20.12) (end 15.39 24.874) (width 0.254) (layer F.Cu) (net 6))
 (segment (start 14.12 18.85) (end 15.39 20.12) (width 0.254) (layer F.Cu) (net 6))
 (segment (start 14.28 21.39) (end 19.2 16.47) (width 0.254) (layer B.Cu) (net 7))
 (segment (start 14.12 21.39) (end 14.28 21.39) (width 0.254) (layer B.Cu) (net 7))
 (segment (start 15.3897 26.0743) (end 15.3897 27.16) (width 0.254) (layer F.Cu) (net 7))
 (segment (start 14.5154 25.2) (end 15.3897 26.0743) (width 0.254) (layer F.Cu) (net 7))
 (segment (start 13.7476 25.2) (end 14.5154 25.2) (width 0.254) (layer F.Cu) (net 7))
 (segment (start 12.9698 24.4222) (end 13.7476 25.2) (width 0.254) (layer F.Cu) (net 7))
 (segment (start 12.9698 22.5402) (end 12.9698 24.4222) (width 0.254) (layer F.Cu) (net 7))
 (segment (start 14.12 21.39) (end 12.9698 22.5402) (width 0.254) (layer F.Cu) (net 7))
 (segment (start 16.406 27.16) (end 15.3897 27.16) (width 0.254) (layer F.Cu) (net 7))
 (via (at 16.8579 24.8656) (size 0.889) (layers F.Cu B.Cu) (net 13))
 (segment (start 16.406 28.43) (end 17.4223 28.43) (width 0.254) (layer F.Cu) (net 13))
 (segment (start 15.0556 24.8656) (end 16.8579 24.8656) (width 0.254) (layer B.Cu) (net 13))
 (segment (start 14.12 23.93) (end 15.0556 24.8656) (width 0.254) (layer B.Cu) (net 13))
 (segment (start 17.4223 25.3651) (end 17.4223 28.43) (width 0.254) (layer F.Cu) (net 13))
 (segment (start 16.9228 24.8656) (end 17.4223 25.3651) (width 0.254) (layer F.Cu) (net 13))
 (segment (start 16.8579 24.8656) (end 16.9228 24.8656) (width 0.254) (layer F.Cu) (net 13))
 (segment (start 15.3897 30.2797) (end 15.3897 30.97) (width 0.254) (layer F.Cu) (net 15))
 (segment (start 14.12 29.01) (end 15.3897 30.2797) (width 0.254) (layer F.Cu) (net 15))
 (segment (start 16.406 30.97) (end 15.3897 30.97) (width 0.254) (layer F.Cu) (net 15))
 (segment (start 14.81 32.24) (end 16.406 32.24) (width 0.254) (layer F.Cu) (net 16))
 (segment (start 14.12 31.55) (end 14.81 32.24) (width 0.254) (layer F.Cu) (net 16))
 (segment (start 25.262 15.3072) (end 25.262 14.6) (width 0.254) (layer F.Cu) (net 4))
 (segment (start 25.2493 15.3199) (end 25.262 15.3072) (width 0.254) (layer F.Cu) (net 4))
 (segment (start 25.2493 16.1) (end 25.2493 15.3199) (width 0.254) (layer F.Cu) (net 4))
 (segment (start 23.962 37.8) (end 23.962 38.7528) (width 0.254) (layer F.Cu) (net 18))
 (segment (start 23.938 38.7768) (end 23.962 38.7528) (width 0.254) (layer F.Cu) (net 18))
 (segment (start 23.938 39.5) (end 23.938 38.7768) (width 0.254) (layer F.Cu) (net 18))
 (segment (start 23.962 37.8) (end 23.2632 37.8) (width 0.254) (layer F.Cu) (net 18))
 (segment (start 23.2632 37.1886) (end 23.2632 37.8) (width 0.254) (layer F.Cu) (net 18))
 (segment (start 22.9217 36.8471) (end 23.2632 37.1886) (width 0.254) (layer F.Cu) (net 18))
 (segment (start 21.1791 36.8471) (end 22.9217 36.8471) (width 0.254) (layer F.Cu) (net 18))
 (segment (start 20.5658 37.4604) (end 21.1791 36.8471) (width 0.254) (layer F.Cu) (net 18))
 (segment (start 20.2843 37.4604) (end 20.5658 37.4604) (width 0.254) (layer F.Cu) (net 18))
 (segment (start 19.2 38.5447) (end 20.2843 37.4604) (width 0.254) (layer F.Cu) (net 18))
 (segment (start 19.2 39.675) (end 19.2 38.5447) (width 0.254) (layer F.Cu) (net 18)))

